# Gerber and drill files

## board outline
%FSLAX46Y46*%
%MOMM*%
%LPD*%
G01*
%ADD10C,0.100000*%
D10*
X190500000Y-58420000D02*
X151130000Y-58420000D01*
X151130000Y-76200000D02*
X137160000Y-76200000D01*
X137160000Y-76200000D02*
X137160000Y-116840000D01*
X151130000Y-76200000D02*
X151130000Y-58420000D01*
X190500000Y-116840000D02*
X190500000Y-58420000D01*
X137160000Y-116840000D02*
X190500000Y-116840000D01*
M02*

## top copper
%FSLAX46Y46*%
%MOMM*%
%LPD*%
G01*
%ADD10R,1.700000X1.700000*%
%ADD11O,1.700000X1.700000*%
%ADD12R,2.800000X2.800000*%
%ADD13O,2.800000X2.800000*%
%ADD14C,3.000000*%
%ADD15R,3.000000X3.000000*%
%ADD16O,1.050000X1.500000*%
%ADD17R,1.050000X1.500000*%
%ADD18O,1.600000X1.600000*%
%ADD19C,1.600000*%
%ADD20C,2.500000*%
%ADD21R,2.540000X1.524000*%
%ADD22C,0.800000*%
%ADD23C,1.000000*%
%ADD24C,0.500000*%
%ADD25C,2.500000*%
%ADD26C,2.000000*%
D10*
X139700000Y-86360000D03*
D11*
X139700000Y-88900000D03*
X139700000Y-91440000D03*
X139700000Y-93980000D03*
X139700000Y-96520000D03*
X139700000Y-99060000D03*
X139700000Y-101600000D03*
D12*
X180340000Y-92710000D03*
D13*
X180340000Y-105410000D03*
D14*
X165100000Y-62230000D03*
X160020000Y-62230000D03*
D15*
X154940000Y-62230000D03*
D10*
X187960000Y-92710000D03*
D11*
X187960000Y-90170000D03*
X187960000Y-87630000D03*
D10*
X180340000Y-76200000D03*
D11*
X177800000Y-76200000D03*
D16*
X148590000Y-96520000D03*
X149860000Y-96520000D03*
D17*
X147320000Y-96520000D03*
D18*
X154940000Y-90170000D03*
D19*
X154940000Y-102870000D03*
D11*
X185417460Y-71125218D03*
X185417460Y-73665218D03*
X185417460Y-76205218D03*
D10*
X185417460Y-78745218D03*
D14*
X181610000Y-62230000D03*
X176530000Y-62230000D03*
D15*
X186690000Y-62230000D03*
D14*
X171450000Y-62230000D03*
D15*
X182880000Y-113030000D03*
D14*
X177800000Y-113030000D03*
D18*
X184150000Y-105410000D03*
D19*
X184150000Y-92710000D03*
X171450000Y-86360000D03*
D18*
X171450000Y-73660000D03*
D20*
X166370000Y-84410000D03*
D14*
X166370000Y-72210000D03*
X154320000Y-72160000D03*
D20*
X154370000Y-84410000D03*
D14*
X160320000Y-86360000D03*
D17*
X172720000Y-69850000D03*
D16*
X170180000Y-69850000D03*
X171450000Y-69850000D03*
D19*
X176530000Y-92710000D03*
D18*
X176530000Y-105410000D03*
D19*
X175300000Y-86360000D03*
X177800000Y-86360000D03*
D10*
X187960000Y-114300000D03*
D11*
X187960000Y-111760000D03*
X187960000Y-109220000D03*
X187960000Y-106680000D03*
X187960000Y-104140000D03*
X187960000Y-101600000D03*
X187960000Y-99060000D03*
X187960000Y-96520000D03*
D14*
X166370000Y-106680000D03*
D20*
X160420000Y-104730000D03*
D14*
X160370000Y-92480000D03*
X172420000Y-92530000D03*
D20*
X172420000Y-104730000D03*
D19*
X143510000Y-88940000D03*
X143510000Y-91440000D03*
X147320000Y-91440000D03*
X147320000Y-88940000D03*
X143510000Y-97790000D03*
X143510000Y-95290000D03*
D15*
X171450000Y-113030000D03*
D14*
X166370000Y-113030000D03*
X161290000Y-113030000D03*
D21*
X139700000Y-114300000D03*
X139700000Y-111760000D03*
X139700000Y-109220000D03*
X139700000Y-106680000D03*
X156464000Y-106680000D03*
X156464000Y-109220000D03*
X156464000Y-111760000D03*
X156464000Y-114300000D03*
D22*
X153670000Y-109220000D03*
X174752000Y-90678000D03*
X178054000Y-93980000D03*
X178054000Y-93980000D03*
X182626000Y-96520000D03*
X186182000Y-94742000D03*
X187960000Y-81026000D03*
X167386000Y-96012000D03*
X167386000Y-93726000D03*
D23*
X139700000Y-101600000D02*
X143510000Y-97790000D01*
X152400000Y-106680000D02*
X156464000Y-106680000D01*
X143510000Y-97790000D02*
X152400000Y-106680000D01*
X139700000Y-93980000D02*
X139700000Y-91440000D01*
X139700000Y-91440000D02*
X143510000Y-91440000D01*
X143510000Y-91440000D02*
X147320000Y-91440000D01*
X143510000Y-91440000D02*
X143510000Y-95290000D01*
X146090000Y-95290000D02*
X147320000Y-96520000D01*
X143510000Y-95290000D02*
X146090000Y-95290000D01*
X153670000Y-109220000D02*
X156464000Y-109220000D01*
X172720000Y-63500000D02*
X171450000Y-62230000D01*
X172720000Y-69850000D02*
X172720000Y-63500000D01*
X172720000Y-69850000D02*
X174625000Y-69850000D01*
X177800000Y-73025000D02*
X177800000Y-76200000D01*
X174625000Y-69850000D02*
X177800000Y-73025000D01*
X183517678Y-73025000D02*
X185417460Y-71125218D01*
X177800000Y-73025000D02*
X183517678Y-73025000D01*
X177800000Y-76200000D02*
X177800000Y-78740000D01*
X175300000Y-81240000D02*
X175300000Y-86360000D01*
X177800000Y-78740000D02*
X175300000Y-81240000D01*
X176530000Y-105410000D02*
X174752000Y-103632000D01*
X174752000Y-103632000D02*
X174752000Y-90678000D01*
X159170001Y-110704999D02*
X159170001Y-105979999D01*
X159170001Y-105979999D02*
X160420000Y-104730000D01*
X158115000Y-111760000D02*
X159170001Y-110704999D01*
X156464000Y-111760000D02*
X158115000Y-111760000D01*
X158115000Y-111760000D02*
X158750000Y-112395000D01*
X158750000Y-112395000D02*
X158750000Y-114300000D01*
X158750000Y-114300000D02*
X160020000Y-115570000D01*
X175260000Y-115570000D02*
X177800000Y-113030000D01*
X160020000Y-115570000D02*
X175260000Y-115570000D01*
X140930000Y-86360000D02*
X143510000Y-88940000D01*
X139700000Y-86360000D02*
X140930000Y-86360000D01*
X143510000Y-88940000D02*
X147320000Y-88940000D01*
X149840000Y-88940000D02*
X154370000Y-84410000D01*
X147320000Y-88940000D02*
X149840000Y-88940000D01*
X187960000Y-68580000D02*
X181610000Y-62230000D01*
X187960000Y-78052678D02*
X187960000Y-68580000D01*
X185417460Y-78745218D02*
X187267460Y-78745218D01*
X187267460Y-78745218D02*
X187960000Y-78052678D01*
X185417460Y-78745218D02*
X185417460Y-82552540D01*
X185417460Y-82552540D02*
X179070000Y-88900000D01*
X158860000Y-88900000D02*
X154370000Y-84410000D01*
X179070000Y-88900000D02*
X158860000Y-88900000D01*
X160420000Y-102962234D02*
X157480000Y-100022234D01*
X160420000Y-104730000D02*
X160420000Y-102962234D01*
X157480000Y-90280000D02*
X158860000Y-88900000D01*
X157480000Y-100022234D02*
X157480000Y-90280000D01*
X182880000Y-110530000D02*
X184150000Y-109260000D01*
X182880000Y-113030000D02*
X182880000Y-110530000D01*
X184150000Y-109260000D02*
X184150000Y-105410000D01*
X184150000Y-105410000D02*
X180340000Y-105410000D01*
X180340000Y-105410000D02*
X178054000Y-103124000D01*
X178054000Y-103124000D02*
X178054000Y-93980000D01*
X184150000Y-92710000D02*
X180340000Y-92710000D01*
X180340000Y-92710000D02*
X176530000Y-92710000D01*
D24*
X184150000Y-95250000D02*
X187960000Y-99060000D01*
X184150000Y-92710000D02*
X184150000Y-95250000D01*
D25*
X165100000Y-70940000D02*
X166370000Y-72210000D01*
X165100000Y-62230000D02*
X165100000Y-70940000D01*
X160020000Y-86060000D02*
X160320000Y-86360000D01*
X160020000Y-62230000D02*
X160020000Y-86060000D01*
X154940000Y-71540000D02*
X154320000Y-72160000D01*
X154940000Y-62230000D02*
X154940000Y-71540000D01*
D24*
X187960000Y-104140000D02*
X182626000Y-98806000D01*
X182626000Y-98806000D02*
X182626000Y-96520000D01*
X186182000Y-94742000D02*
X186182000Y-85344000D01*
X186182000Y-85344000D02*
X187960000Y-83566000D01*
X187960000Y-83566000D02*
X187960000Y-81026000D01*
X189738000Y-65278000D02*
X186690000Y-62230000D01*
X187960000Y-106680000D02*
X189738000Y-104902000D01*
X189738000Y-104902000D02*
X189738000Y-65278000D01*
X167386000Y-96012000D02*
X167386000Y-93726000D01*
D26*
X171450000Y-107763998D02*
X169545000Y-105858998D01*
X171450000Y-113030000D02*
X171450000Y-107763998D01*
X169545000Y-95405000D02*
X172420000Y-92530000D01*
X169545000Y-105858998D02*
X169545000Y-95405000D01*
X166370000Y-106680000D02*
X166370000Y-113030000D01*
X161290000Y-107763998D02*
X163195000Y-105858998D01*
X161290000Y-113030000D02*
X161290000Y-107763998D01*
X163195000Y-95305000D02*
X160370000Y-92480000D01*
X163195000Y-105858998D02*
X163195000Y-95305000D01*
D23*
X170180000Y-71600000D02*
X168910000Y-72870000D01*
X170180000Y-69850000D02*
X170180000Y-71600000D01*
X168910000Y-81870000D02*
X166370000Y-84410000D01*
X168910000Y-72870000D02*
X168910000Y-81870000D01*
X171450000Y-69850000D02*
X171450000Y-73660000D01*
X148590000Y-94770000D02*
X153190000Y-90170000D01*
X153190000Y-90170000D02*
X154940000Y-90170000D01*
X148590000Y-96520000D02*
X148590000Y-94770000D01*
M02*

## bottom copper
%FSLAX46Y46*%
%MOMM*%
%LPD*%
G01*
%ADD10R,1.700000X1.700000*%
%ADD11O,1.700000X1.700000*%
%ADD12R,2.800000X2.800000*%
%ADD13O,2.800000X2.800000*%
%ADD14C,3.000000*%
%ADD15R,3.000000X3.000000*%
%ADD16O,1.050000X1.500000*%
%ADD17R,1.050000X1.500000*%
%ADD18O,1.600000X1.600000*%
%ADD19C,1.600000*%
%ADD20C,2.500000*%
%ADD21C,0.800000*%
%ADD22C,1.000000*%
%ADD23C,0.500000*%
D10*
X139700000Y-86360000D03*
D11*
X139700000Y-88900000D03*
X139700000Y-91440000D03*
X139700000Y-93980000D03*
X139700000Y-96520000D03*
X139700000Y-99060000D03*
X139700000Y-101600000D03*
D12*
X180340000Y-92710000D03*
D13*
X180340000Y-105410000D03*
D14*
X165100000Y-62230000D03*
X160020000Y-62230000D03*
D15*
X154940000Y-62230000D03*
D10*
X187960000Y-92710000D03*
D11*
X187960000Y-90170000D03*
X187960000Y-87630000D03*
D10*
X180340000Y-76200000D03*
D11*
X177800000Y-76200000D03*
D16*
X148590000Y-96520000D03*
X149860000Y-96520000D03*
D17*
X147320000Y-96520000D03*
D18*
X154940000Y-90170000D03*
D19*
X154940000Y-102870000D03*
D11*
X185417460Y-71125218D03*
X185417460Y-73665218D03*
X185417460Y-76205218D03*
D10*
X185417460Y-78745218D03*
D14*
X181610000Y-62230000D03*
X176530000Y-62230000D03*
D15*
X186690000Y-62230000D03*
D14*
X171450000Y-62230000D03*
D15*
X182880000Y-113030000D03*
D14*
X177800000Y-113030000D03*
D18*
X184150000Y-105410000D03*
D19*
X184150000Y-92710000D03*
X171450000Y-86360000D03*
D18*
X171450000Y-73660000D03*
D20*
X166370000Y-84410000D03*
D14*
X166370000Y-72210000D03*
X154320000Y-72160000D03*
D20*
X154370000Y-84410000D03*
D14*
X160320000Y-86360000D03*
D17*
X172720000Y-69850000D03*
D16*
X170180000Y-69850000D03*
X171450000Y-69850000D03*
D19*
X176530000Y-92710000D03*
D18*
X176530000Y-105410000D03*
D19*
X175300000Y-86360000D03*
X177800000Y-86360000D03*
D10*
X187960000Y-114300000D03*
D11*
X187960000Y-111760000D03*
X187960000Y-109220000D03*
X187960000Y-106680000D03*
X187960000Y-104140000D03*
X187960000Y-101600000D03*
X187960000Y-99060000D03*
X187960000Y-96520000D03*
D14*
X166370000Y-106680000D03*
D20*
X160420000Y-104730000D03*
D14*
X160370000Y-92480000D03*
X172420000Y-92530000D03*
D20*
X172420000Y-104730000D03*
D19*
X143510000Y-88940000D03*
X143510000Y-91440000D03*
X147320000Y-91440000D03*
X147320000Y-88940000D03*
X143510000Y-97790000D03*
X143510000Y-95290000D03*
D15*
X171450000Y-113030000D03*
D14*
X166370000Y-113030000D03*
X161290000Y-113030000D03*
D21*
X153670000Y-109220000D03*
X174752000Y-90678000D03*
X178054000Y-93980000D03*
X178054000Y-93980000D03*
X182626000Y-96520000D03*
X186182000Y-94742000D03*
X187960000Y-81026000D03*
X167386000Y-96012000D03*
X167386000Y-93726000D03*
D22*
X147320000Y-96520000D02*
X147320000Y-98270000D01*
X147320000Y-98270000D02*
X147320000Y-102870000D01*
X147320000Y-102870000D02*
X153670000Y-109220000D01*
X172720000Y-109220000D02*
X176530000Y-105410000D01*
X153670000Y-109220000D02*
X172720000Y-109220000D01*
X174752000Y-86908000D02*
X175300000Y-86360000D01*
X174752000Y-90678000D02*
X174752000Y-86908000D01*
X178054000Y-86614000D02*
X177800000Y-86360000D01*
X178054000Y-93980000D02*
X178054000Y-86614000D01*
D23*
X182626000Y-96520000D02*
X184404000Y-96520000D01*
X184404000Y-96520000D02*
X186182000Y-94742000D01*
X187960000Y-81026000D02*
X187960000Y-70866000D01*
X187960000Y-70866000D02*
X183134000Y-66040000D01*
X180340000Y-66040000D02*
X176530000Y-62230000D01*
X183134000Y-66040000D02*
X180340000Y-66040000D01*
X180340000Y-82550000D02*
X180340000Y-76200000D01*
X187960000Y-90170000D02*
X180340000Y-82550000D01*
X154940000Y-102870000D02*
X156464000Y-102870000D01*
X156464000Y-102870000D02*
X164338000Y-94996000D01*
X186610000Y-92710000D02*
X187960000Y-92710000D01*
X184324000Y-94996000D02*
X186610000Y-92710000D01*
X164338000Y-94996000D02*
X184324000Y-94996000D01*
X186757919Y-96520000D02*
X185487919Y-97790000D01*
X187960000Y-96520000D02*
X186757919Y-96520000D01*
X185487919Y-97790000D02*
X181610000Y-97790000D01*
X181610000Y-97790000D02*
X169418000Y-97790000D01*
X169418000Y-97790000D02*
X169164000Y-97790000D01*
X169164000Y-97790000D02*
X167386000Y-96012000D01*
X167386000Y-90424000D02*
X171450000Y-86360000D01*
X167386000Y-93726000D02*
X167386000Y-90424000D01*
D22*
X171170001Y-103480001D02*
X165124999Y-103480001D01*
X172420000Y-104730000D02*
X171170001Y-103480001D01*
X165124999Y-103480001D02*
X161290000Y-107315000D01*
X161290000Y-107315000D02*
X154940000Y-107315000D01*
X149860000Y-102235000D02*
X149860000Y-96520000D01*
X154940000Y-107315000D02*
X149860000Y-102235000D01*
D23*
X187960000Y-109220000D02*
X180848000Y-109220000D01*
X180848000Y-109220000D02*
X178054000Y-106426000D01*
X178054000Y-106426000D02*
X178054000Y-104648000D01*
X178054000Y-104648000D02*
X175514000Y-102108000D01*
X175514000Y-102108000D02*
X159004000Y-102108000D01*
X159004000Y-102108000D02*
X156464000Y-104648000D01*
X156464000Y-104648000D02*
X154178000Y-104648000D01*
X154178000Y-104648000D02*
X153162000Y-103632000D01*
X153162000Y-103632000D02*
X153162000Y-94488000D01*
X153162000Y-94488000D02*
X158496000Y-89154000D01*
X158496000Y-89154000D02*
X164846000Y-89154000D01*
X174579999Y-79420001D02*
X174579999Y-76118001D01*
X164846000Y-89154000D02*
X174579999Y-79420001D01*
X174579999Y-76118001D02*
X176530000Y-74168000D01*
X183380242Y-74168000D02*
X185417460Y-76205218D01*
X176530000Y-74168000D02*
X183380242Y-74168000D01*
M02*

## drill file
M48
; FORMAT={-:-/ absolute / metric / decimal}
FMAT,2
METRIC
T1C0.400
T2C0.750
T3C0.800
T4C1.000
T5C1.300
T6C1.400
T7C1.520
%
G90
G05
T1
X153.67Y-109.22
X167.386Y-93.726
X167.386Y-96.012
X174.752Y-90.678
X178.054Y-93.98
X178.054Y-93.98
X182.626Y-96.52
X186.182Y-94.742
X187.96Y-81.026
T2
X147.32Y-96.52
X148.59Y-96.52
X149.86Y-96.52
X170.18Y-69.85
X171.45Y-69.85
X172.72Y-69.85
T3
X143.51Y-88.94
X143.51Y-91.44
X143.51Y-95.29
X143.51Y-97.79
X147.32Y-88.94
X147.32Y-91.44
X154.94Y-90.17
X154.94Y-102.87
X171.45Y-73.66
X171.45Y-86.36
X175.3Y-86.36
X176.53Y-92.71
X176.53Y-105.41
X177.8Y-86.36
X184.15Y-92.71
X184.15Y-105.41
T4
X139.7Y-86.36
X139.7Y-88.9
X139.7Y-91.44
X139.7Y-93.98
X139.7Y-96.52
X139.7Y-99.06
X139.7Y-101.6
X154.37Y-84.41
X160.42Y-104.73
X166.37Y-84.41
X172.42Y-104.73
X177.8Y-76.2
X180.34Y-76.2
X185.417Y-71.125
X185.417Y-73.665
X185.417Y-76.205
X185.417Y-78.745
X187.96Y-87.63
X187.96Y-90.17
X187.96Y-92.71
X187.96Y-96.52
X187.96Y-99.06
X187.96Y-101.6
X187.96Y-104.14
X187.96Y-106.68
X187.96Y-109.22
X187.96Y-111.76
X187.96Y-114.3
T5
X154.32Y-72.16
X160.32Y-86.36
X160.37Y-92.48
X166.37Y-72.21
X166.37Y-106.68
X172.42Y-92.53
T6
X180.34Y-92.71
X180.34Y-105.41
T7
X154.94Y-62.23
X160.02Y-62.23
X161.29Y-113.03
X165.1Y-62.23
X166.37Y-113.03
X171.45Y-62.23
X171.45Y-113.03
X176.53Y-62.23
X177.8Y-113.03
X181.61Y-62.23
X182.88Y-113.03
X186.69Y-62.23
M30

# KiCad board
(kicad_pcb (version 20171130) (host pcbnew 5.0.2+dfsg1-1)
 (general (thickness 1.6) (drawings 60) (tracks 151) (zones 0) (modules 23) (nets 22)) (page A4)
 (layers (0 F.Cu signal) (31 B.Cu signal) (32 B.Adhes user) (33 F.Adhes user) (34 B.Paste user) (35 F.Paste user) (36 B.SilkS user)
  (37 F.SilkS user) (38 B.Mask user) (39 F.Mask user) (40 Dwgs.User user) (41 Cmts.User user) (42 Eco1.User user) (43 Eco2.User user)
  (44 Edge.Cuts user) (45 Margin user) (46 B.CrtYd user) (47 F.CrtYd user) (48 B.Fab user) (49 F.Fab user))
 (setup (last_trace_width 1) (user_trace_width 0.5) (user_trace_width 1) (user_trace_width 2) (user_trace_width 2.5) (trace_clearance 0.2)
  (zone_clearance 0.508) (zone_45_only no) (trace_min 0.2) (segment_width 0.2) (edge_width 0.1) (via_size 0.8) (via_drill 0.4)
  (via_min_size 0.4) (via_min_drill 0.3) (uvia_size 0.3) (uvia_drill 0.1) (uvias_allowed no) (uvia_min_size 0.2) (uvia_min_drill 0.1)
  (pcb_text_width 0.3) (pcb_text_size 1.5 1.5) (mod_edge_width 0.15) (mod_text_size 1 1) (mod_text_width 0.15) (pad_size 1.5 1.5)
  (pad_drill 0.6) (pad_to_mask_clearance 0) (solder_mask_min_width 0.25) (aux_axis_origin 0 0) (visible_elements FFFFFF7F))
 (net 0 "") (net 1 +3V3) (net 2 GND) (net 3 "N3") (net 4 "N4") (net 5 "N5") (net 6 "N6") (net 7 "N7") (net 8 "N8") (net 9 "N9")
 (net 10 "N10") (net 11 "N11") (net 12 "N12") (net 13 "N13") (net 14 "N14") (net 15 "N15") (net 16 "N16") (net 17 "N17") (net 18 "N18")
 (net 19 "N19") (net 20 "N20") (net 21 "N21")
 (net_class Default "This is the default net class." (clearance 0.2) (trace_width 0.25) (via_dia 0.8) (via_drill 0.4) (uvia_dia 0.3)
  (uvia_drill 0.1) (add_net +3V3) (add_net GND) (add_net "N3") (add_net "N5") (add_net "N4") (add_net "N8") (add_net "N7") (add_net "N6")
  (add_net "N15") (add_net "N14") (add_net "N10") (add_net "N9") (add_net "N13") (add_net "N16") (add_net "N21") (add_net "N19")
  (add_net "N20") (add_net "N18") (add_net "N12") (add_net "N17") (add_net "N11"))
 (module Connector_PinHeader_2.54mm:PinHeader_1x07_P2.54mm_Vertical (layer F.Cu) (at 139.7 86.36)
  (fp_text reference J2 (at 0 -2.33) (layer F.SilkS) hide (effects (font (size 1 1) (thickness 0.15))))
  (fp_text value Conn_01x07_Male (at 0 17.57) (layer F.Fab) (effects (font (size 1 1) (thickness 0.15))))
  (pad 1 thru_hole rect (at 0 0) (size 1.7 1.7) (drill 1) (layers *.Cu *.Mask) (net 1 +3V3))
  (pad 2 thru_hole oval (at 0 2.54) (size 1.7 1.7) (drill 1) (layers *.Cu *.Mask))
  (pad 3 thru_hole oval (at 0 5.08) (size 1.7 1.7) (drill 1) (layers *.Cu *.Mask) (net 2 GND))
  (pad 4 thru_hole oval (at 0 7.62) (size 1.7 1.7) (drill 1) (layers *.Cu *.Mask) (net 2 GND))
  (pad 5 thru_hole oval (at 0 10.16) (size 1.7 1.7) (drill 1) (layers *.Cu *.Mask))
  (pad 6 thru_hole oval (at 0 12.7) (size 1.7 1.7) (drill 1) (layers *.Cu *.Mask))
  (pad 7 thru_hole oval (at 0 15.24) (size 1.7 1.7) (drill 1) (layers *.Cu *.Mask) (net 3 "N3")))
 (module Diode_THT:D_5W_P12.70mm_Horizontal (layer F.Cu) (at 180.34 92.71 270)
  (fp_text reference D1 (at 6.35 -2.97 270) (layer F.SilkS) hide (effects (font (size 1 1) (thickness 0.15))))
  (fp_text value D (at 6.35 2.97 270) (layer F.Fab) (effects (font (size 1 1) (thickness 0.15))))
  (pad 1 thru_hole rect (at 0 0 270) (size 2.8 2.8) (drill 1.4) (layers *.Cu *.Mask) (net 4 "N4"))
  (pad 2 thru_hole oval (at 12.7 0 270) (size 2.8 2.8) (drill 1.4) (layers *.Cu *.Mask) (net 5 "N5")))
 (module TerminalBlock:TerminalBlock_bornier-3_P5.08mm (layer F.Cu) (at 154.94 62.23)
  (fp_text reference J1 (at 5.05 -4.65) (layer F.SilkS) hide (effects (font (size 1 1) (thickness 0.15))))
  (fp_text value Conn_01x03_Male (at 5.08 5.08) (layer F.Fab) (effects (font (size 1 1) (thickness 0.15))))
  (pad 3 thru_hole circle (at 10.16 0) (size 3 3) (drill 1.52) (layers *.Cu *.Mask) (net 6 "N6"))
  (pad 2 thru_hole circle (at 5.08 0) (size 3 3) (drill 1.52) (layers *.Cu *.Mask) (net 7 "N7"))
  (pad 1 thru_hole rect (at 0 0) (size 3 3) (drill 1.52) (layers *.Cu *.Mask) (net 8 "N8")))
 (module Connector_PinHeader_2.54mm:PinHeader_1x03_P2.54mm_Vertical (layer F.Cu) (at 187.96 92.71 180)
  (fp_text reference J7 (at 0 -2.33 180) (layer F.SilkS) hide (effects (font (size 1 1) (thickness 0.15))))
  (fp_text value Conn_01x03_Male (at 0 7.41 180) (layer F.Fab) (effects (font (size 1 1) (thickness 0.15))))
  (pad 1 thru_hole rect (at 0 0 180) (size 1.7 1.7) (drill 1) (layers *.Cu *.Mask) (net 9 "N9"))
  (pad 2 thru_hole oval (at 0 2.54 180) (size 1.7 1.7) (drill 1) (layers *.Cu *.Mask) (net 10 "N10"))
  (pad 3 thru_hole oval (at 0 5.08 180) (size 1.7 1.7) (drill 1) (layers *.Cu *.Mask)))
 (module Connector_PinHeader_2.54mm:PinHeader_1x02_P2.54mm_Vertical (layer F.Cu) (at 180.34 76.2 270)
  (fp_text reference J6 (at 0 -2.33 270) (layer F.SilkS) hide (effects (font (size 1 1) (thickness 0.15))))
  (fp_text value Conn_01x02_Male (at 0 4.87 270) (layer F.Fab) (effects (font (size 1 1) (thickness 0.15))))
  (pad 1 thru_hole rect (at 0 0 270) (size 1.7 1.7) (drill 1) (layers *.Cu *.Mask) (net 10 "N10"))
  (pad 2 thru_hole oval (at 0 2.54 270) (size 1.7 1.7) (drill 1) (layers *.Cu *.Mask) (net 2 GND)))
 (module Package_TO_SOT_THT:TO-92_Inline (layer F.Cu) (at 147.32 96.52)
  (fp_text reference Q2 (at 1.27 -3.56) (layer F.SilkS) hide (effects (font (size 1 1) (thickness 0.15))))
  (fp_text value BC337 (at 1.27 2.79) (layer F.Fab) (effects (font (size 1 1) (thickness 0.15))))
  (pad 2 thru_hole oval (at 1.27 0) (size 1.05 1.5) (drill 0.75) (layers *.Cu *.Mask) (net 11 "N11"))
  (pad 3 thru_hole oval (at 2.54 0) (size 1.05 1.5) (drill 0.75) (layers *.Cu *.Mask) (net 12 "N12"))
  (pad 1 thru_hole rect (at 0 0) (size 1.05 1.5) (drill 0.75) (layers *.Cu *.Mask) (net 2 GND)))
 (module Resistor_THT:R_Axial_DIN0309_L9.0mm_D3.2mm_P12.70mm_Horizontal (layer F.Cu) (at 154.94 102.87 90)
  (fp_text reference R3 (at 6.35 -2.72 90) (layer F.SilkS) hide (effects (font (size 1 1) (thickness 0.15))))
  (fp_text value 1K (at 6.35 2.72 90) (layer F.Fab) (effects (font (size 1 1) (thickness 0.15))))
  (pad 2 thru_hole oval (at 12.7 0 90) (size 1.6 1.6) (drill 0.8) (layers *.Cu *.Mask) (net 11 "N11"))
  (pad 1 thru_hole circle (at 0 0 90) (size 1.6 1.6) (drill 0.8) (layers *.Cu *.Mask) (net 9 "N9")))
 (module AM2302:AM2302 (layer F.Cu) (at 185.42 74.93 90)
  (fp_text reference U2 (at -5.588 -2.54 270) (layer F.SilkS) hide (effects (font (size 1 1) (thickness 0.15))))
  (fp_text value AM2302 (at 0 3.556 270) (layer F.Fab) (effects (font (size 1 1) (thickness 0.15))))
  (pad 4 thru_hole oval (at 3.804782 -0.00254 180) (size 1.7 1.7) (drill 1) (layers *.Cu *.Mask) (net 2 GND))
  (pad 3 thru_hole oval (at 1.264782 -0.00254 180) (size 1.7 1.7) (drill 1) (layers *.Cu *.Mask))
  (pad 2 thru_hole oval (at -1.275218 -0.00254 180) (size 1.7 1.7) (drill 1) (layers *.Cu *.Mask) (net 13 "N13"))
  (pad 1 thru_hole rect (at -3.815218 -0.00254) (size 1.7 1.7) (drill 1) (layers *.Cu *.Mask) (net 1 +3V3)))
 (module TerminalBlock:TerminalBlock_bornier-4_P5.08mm (layer F.Cu) (at 186.69 62.23 180)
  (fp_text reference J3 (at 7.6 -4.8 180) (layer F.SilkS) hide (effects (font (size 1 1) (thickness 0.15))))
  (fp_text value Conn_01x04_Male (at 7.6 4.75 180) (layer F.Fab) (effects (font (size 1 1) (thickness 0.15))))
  (pad 2 thru_hole circle (at 5.08 0 180) (size 3 3) (drill 1.52) (layers *.Cu *.Mask) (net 1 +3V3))
  (pad 3 thru_hole circle (at 10.16 0 180) (size 3 3) (drill 1.52) (layers *.Cu *.Mask) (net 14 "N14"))
  (pad 1 thru_hole rect (at 0 0 180) (size 3 3) (drill 1.52) (layers *.Cu *.Mask) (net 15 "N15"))
  (pad 4 thru_hole circle (at 15.24 0 180) (size 3 3) (drill 1.52) (layers *.Cu *.Mask) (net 2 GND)))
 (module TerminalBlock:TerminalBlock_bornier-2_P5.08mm (layer F.Cu) (at 182.88 113.03 180)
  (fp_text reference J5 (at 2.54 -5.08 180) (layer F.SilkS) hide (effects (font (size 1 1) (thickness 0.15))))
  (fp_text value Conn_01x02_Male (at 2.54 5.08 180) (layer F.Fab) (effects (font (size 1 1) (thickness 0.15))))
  (pad 1 thru_hole rect (at 0 0 180) (size 3 3) (drill 1.52) (layers *.Cu *.Mask) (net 5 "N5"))
  (pad 2 thru_hole circle (at 5.08 0 180) (size 3 3) (drill 1.52) (layers *.Cu *.Mask) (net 1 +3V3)))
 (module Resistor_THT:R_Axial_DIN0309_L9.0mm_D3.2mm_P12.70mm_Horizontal (layer F.Cu) (at 184.15 92.71 270)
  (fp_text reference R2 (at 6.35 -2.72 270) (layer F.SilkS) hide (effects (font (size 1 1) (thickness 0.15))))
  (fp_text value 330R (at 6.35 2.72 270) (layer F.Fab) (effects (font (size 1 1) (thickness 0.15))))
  (pad 2 thru_hole oval (at 12.7 0 270) (size 1.6 1.6) (drill 0.8) (layers *.Cu *.Mask) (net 5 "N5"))
  (pad 1 thru_hole circle (at 0 0 270) (size 1.6 1.6) (drill 0.8) (layers *.Cu *.Mask) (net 4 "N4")))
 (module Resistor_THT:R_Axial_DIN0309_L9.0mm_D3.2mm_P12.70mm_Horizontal (layer F.Cu) (at 171.45 86.36 90)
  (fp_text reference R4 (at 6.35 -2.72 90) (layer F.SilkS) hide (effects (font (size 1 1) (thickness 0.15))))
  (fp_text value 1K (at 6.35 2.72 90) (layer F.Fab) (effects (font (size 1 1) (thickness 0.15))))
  (pad 1 thru_hole circle (at 0 0 90) (size 1.6 1.6) (drill 0.8) (layers *.Cu *.Mask) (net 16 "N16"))
  (pad 2 thru_hole oval (at 12.7 0 90) (size 1.6 1.6) (drill 0.8) (layers *.Cu *.Mask) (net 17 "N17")))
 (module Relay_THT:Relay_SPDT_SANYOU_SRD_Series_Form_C (layer F.Cu) (at 160.32 86.36 90)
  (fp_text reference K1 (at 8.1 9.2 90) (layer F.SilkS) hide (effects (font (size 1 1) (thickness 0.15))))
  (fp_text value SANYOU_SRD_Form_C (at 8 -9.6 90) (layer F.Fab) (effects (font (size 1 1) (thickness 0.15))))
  (pad 2 thru_hole circle (at 1.95 6.05 180) (size 2.5 2.5) (drill 1) (layers *.Cu *.Mask) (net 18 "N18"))
  (pad 3 thru_hole circle (at 14.15 6.05 180) (size 3 3) (drill 1.3) (layers *.Cu *.Mask) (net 6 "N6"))
  (pad 4 thru_hole circle (at 14.2 -6 180) (size 3 3) (drill 1.3) (layers *.Cu *.Mask) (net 8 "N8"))
  (pad 5 thru_hole circle (at 1.95 -5.95 180) (size 2.5 2.5) (drill 1) (layers *.Cu *.Mask) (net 1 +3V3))
  (pad 1 thru_hole circle (at 0 0 180) (size 3 3) (drill 1.3) (layers *.Cu *.Mask) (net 7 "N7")))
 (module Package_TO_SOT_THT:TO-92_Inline (layer F.Cu) (at 172.72 69.85 180)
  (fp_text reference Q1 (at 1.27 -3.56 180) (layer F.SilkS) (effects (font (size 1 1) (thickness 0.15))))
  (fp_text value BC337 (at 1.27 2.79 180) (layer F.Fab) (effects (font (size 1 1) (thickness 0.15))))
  (pad 1 thru_hole rect (at 0 0 180) (size 1.05 1.5) (drill 0.75) (layers *.Cu *.Mask) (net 2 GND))
  (pad 3 thru_hole oval (at 2.54 0 180) (size 1.05 1.5) (drill 0.75) (layers *.Cu *.Mask) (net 18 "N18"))
  (pad 2 thru_hole oval (at 1.27 0 180) (size 1.05 1.5) (drill 0.75) (layers *.Cu *.Mask) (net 17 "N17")))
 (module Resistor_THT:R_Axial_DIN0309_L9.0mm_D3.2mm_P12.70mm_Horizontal (layer F.Cu) (at 176.53 92.71 270)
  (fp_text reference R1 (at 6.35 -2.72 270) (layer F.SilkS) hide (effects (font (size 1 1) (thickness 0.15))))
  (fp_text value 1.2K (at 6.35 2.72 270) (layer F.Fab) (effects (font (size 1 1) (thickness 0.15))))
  (pad 1 thru_hole circle (at 0 0 270) (size 1.6 1.6) (drill 0.8) (layers *.Cu *.Mask) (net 4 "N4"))
  (pad 2 thru_hole oval (at 12.7 0 270) (size 1.6 1.6) (drill 0.8) (layers *.Cu *.Mask) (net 2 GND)))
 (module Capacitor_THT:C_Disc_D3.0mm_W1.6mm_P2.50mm (layer F.Cu) (at 177.8 86.36 180)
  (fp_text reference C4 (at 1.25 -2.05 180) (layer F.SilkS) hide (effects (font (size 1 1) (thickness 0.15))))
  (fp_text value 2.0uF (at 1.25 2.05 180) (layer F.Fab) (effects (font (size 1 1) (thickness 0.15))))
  (pad 2 thru_hole circle (at 2.5 0 180) (size 1.6 1.6) (drill 0.8) (layers *.Cu *.Mask) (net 2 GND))
  (pad 1 thru_hole circle (at 0 0 180) (size 1.6 1.6) (drill 0.8) (layers *.Cu *.Mask) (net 5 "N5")))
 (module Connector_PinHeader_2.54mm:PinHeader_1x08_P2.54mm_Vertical (layer F.Cu) (at 187.96 114.3 180)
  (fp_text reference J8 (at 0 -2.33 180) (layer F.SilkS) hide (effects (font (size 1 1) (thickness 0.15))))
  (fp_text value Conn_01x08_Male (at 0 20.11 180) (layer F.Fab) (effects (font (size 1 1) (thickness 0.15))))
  (pad 1 thru_hole rect (at 0 0 180) (size 1.7 1.7) (drill 1) (layers *.Cu *.Mask))
  (pad 2 thru_hole oval (at 0 2.54 180) (size 1.7 1.7) (drill 1) (layers *.Cu *.Mask))
  (pad 3 thru_hole oval (at 0 5.08 180) (size 1.7 1.7) (drill 1) (layers *.Cu *.Mask) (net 13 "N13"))
  (pad 4 thru_hole oval (at 0 7.62 180) (size 1.7 1.7) (drill 1) (layers *.Cu *.Mask) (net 15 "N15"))
  (pad 5 thru_hole oval (at 0 10.16 180) (size 1.7 1.7) (drill 1) (layers *.Cu *.Mask) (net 14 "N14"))
  (pad 6 thru_hole oval (at 0 12.7 180) (size 1.7 1.7) (drill 1) (layers *.Cu *.Mask))
  (pad 7 thru_hole oval (at 0 15.24 180) (size 1.7 1.7) (drill 1) (layers *.Cu *.Mask) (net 4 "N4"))
  (pad 8 thru_hole oval (at 0 17.78 180) (size 1.7 1.7) (drill 1) (layers *.Cu *.Mask) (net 16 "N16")))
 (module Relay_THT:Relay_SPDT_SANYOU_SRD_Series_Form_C (layer F.Cu) (at 166.37 106.68 90)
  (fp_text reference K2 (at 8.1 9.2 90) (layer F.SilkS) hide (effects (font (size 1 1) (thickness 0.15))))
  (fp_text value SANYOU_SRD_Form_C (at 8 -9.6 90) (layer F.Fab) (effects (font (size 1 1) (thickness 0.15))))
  (pad 1 thru_hole circle (at 0 0 180) (size 3 3) (drill 1.3) (layers *.Cu *.Mask) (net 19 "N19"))
  (pad 5 thru_hole circle (at 1.95 -5.95 180) (size 2.5 2.5) (drill 1) (layers *.Cu *.Mask) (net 1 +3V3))
  (pad 4 thru_hole circle (at 14.2 -6 180) (size 3 3) (drill 1.3) (layers *.Cu *.Mask) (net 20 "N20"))
  (pad 3 thru_hole circle (at 14.15 6.05 180) (size 3 3) (drill 1.3) (layers *.Cu *.Mask) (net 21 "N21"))
  (pad 2 thru_hole circle (at 1.95 6.05 180) (size 2.5 2.5) (drill 1) (layers *.Cu *.Mask) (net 12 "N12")))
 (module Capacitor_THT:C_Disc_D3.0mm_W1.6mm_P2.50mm (layer F.Cu) (at 143.51 88.94 270)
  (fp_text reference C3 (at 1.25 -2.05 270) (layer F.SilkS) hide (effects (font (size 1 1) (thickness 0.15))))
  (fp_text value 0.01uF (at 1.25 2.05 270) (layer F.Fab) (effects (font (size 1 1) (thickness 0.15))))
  (pad 1 thru_hole circle (at 0 0 270) (size 1.6 1.6) (drill 0.8) (layers *.Cu *.Mask) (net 1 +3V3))
  (pad 2 thru_hole circle (at 2.5 0 270) (size 1.6 1.6) (drill 0.8) (layers *.Cu *.Mask) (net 2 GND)))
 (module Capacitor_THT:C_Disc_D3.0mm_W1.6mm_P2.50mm (layer F.Cu) (at 147.32 88.94 270)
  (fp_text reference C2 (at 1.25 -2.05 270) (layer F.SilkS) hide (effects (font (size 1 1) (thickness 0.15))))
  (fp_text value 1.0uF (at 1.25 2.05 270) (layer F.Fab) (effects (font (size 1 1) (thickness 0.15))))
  (pad 2 thru_hole circle (at 2.5 0 270) (size 1.6 1.6) (drill 0.8) (layers *.Cu *.Mask) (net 2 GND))
  (pad 1 thru_hole circle (at 0 0 270) (size 1.6 1.6) (drill 0.8) (layers *.Cu *.Mask) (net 1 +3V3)))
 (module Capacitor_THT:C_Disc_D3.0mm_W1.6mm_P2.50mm (layer F.Cu) (at 143.51 97.79 90)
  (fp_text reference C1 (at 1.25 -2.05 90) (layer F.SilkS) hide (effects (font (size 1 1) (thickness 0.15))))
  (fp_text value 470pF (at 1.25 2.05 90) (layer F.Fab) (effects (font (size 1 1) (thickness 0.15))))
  (pad 1 thru_hole circle (at 0 0 90) (size 1.6 1.6) (drill 0.8) (layers *.Cu *.Mask) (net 3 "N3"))
  (pad 2 thru_hole circle (at 2.5 0 90) (size 1.6 1.6) (drill 0.8) (layers *.Cu *.Mask) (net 2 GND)))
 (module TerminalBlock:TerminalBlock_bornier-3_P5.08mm (layer F.Cu) (at 171.45 113.03 180)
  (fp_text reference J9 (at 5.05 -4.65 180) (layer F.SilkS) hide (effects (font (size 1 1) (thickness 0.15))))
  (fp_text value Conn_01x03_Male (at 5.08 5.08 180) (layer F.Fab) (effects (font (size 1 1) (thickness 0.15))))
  (pad 1 thru_hole rect (at 0 0 180) (size 3 3) (drill 1.52) (layers *.Cu *.Mask) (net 21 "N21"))
  (pad 2 thru_hole circle (at 5.08 0 180) (size 3 3) (drill 1.52) (layers *.Cu *.Mask) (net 19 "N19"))
  (pad 3 thru_hole circle (at 10.16 0 180) (size 3 3) (drill 1.52) (layers *.Cu *.Mask) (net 20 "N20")))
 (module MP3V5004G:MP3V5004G (layer F.Cu) (at 148.082 110.49)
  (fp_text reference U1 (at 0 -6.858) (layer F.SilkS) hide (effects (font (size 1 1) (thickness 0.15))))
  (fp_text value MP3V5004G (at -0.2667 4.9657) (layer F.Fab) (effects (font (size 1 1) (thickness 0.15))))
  (pad 8 smd rect (at -8.382 3.81) (size 2.54 1.524) (layers F.Cu F.Paste F.Mask))
  (pad 7 smd rect (at -8.382 1.27) (size 2.54 1.524) (layers F.Cu F.Paste F.Mask))
  (pad 6 smd rect (at -8.382 -1.27) (size 2.54 1.524) (layers F.Cu F.Paste F.Mask))
  (pad 5 smd rect (at -8.382 -3.81) (size 2.54 1.524) (layers F.Cu F.Paste F.Mask))
  (pad 4 smd rect (at 8.382 -3.81) (size 2.54 1.524) (layers F.Cu F.Paste F.Mask) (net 3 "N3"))
  (pad 3 smd rect (at 8.382 -1.27) (size 2.54 1.524) (layers F.Cu F.Paste F.Mask) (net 2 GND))
  (pad 2 smd rect (at 8.382 1.27) (size 2.54 1.524) (layers F.Cu F.Paste F.Mask) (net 1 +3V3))
  (pad 1 smd rect (at 8.382 3.81) (size 2.54 1.524) (layers F.Cu F.Paste F.Mask)))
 (gr_line (start 190.5 58.42) (end 151.13 58.42) (layer Edge.Cuts) (width 0.1))
 (gr_line (start 151.13 76.2) (end 137.16 76.2) (layer Edge.Cuts) (width 0.1))
 (gr_line (start 137.16 76.2) (end 137.16 116.84) (layer Edge.Cuts) (width 0.1))
 (gr_line (start 151.13 76.2) (end 151.13 58.42) (layer Edge.Cuts) (width 0.1))
 (gr_line (start 190.5 116.84) (end 190.5 58.42) (layer Edge.Cuts) (width 0.1))
 (gr_line (start 137.16 116.84) (end 190.5 116.84) (layer Edge.Cuts) (width 0.1))
 (segment (start 139.7 101.6) (end 143.51 97.79) (width 1) (layer F.Cu) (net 3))
 (segment (start 152.4 106.68) (end 156.464 106.68) (width 1) (layer F.Cu) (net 3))
 (segment (start 143.51 97.79) (end 152.4 106.68) (width 1) (layer F.Cu) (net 3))
 (segment (start 139.7 93.98) (end 139.7 91.44) (width 1) (layer F.Cu) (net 2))
 (segment (start 139.7 91.44) (end 143.51 91.44) (width 1) (layer F.Cu) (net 2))
 (segment (start 143.51 91.44) (end 147.32 91.44) (width 1) (layer F.Cu) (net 2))
 (segment (start 143.51 91.44) (end 143.51 95.29) (width 1) (layer F.Cu) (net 2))
 (segment (start 146.09 95.29) (end 147.32 96.52) (width 1) (layer F.Cu) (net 2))
 (segment (start 143.51 95.29) (end 146.09 95.29) (width 1) (layer F.Cu) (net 2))
 (segment (start 147.32 96.52) (end 147.32 98.27) (width 1) (layer B.Cu) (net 2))
 (segment (start 147.32 98.27) (end 147.32 102.87) (width 1) (layer B.Cu) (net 2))
 (via (at 153.67 109.22) (size 0.8) (drill 0.4) (layers F.Cu B.Cu) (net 2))
 (segment (start 147.32 102.87) (end 153.67 109.22) (width 1) (layer B.Cu) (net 2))
 (segment (start 153.67 109.22) (end 156.464 109.22) (width 1) (layer F.Cu) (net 2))
 (segment (start 172.72 109.22) (end 176.53 105.41) (width 1) (layer B.Cu) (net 2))
 (segment (start 153.67 109.22) (end 172.72 109.22) (width 1) (layer B.Cu) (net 2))
 (segment (start 172.72 63.5) (end 171.45 62.23) (width 1) (layer F.Cu) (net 2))
 (segment (start 172.72 69.85) (end 172.72 63.5) (width 1) (layer F.Cu) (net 2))
 (segment (start 172.72 69.85) (end 174.625 69.85) (width 1) (layer F.Cu) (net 2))
 (segment (start 177.8 73.025) (end 177.8 76.2) (width 1) (layer F.Cu) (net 2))
 (segment (start 174.625 69.85) (end 177.8 73.025) (width 1) (layer F.Cu) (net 2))
 (segment (start 183.517678 73.025) (end 185.41746 71.125218) (width 1) (layer F.Cu) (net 2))
 (segment (start 177.8 73.025) (end 183.517678 73.025) (width 1) (layer F.Cu) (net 2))
 (segment (start 177.8 76.2) (end 177.8 78.74) (width 1) (layer F.Cu) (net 2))
 (segment (start 175.3 81.24) (end 175.3 86.36) (width 1) (layer F.Cu) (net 2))
 (segment (start 177.8 78.74) (end 175.3 81.24) (width 1) (layer F.Cu) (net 2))
 (segment (start 176.53 105.41) (end 174.752 103.632) (width 1) (layer F.Cu) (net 2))
 (via (at 174.752 90.678) (size 0.8) (drill 0.4) (layers F.Cu B.Cu) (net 2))
 (segment (start 174.752 103.632) (end 174.752 90.678) (width 1) (layer F.Cu) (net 2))
 (segment (start 174.752 86.908) (end 175.3 86.36) (width 1) (layer B.Cu) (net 2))
 (segment (start 174.752 90.678) (end 174.752 86.908) (width 1) (layer B.Cu) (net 2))
 (segment (start 159.170001 110.704999) (end 159.170001 105.979999) (width 1) (layer F.Cu) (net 1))
 (segment (start 159.170001 105.979999) (end 160.42 104.73) (width 1) (layer F.Cu) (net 1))
 (segment (start 158.115 111.76) (end 159.170001 110.704999) (width 1) (layer F.Cu) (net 1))
 (segment (start 156.464 111.76) (end 158.115 111.76) (width 1) (layer F.Cu) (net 1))
 (segment (start 158.115 111.76) (end 158.75 112.395) (width 1) (layer F.Cu) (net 1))
 (segment (start 158.75 112.395) (end 158.75 114.3) (width 1) (layer F.Cu) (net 1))
 (segment (start 158.75 114.3) (end 160.02 115.57) (width 1) (layer F.Cu) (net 1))
 (segment (start 175.26 115.57) (end 177.8 113.03) (width 1) (layer F.Cu) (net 1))
 (segment (start 160.02 115.57) (end 175.26 115.57) (width 1) (layer F.Cu) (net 1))
 (segment (start 140.93 86.36) (end 143.51 88.94) (width 1) (layer F.Cu) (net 1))
 (segment (start 139.7 86.36) (end 140.93 86.36) (width 1) (layer F.Cu) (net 1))
 (segment (start 143.51 88.94) (end 147.32 88.94) (width 1) (layer F.Cu) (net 1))
 (segment (start 149.84 88.94) (end 154.37 84.41) (width 1) (layer F.Cu) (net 1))
 (segment (start 147.32 88.94) (end 149.84 88.94) (width 1) (layer F.Cu) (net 1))
 (segment (start 187.96 68.58) (end 181.61 62.23) (width 1) (layer F.Cu) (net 1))
 (segment (start 187.96 78.052678) (end 187.96 68.58) (width 1) (layer F.Cu) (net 1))
 (segment (start 185.41746 78.745218) (end 187.26746 78.745218) (width 1) (layer F.Cu) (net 1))
 (segment (start 187.26746 78.745218) (end 187.96 78.052678) (width 1) (layer F.Cu) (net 1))
 (segment (start 185.41746 78.745218) (end 185.41746 82.55254) (width 1) (layer F.Cu) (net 1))
 (segment (start 185.41746 82.55254) (end 179.07 88.9) (width 1) (layer F.Cu) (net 1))
 (segment (start 158.86 88.9) (end 154.37 84.41) (width 1) (layer F.Cu) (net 1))
 (segment (start 179.07 88.9) (end 158.86 88.9) (width 1) (layer F.Cu) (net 1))
 (segment (start 160.42 102.962234) (end 157.48 100.022234) (width 1) (layer F.Cu) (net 1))
 (segment (start 160.42 104.73) (end 160.42 102.962234) (width 1) (layer F.Cu) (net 1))
 (segment (start 157.48 90.28) (end 158.86 88.9) (width 1) (layer F.Cu) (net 1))
 (segment (start 157.48 100.022234) (end 157.48 90.28) (width 1) (layer F.Cu) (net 1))
 (segment (start 182.88 110.53) (end 184.15 109.26) (width 1) (layer F.Cu) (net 5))
 (segment (start 182.88 113.03) (end 182.88 110.53) (width 1) (layer F.Cu) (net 5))
 (segment (start 184.15 109.26) (end 184.15 105.41) (width 1) (layer F.Cu) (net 5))
 (segment (start 184.15 105.41) (end 180.34 105.41) (width 1) (layer F.Cu) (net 5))
 (via (at 178.054 93.98) (size 0.8) (drill 0.4) (layers F.Cu B.Cu) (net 5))
 (segment (start 180.34 105.41) (end 178.054 103.124) (width 1) (layer F.Cu) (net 5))
 (segment (start 178.054 103.124) (end 178.054 93.98) (width 1) (layer F.Cu) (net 5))
 (via (at 178.054 93.98) (size 0.8) (drill 0.4) (layers F.Cu B.Cu) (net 5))
 (segment (start 178.054 86.614) (end 177.8 86.36) (width 1) (layer B.Cu) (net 5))
 (segment (start 178.054 93.98) (end 178.054 86.614) (width 1) (layer B.Cu) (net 5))
 (segment (start 184.15 92.71) (end 180.34 92.71) (width 1) (layer F.Cu) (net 4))
 (segment (start 180.34 92.71) (end 176.53 92.71) (width 1) (layer F.Cu) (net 4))
 (segment (start 184.15 95.25) (end 187.96 99.06) (width 0.5) (layer F.Cu) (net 4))
 (segment (start 184.15 92.71) (end 184.15 95.25) (width 0.5) (layer F.Cu) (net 4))
 (segment (start 165.1 70.94) (end 166.37 72.21) (width 2.5) (layer F.Cu) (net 6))
 (segment (start 165.1 62.23) (end 165.1 70.94) (width 2.5) (layer F.Cu) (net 6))
 (segment (start 160.02 86.06) (end 160.32 86.36) (width 2.5) (layer F.Cu) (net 7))
 (segment (start 160.02 62.23) (end 160.02 86.06) (width 2.5) (layer F.Cu) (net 7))
 (segment (start 154.94 71.54) (end 154.32 72.16) (width 2.5) (layer F.Cu) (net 8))
 (segment (start 154.94 62.23) (end 154.94 71.54) (width 2.5) (layer F.Cu) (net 8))
 (segment (start 187.96 104.14) (end 182.626 98.806) (width 0.5) (layer F.Cu) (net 14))
 (via (at 182.626 96.52) (size 0.8) (drill 0.4) (layers F.Cu B.Cu) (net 14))
 (segment (start 182.626 98.806) (end 182.626 96.52) (width 0.5) (layer F.Cu) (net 14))
 (via (at 186.182 94.742) (size 0.8) (drill 0.4) (layers F.Cu B.Cu) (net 14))
 (segment (start 182.626 96.52) (end 184.404 96.52) (width 0.5) (layer B.Cu) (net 14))
 (segment (start 184.404 96.52) (end 186.182 94.742) (width 0.5) (layer B.Cu) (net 14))
 (segment (start 186.182 94.742) (end 186.182 85.344) (width 0.5) (layer F.Cu) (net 14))
 (segment (start 186.182 85.344) (end 187.96 83.566) (width 0.5) (layer F.Cu) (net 14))
 (via (at 187.96 81.026) (size 0.8) (drill 0.4) (layers F.Cu B.Cu) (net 14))
 (segment (start 187.96 83.566) (end 187.96 81.026) (width 0.5) (layer F.Cu) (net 14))
 (segment (start 187.96 81.026) (end 187.96 70.866) (width 0.5) (layer B.Cu) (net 14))
 (segment (start 187.96 70.866) (end 183.134 66.04) (width 0.5) (layer B.Cu) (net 14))
 (segment (start 180.34 66.04) (end 176.53 62.23) (width 0.5) (layer B.Cu) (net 14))
 (segment (start 183.134 66.04) (end 180.34 66.04) (width 0.5) (layer B.Cu) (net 14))
 (segment (start 189.738 65.278) (end 186.69 62.23) (width 0.5) (layer F.Cu) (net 15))
 (segment (start 187.96 106.68) (end 189.738 104.902) (width 0.5) (layer F.Cu) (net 15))
 (segment (start 189.738 104.902) (end 189.738 65.278) (width 0.5) (layer F.Cu) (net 15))
 (segment (start 180.34 82.55) (end 180.34 76.2) (width 0.5) (layer B.Cu) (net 10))
 (segment (start 187.96 90.17) (end 180.34 82.55) (width 0.5) (layer B.Cu) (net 10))
 (segment (start 154.94 102.87) (end 156.464 102.87) (width 0.5) (layer B.Cu) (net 9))
 (segment (start 156.464 102.87) (end 164.338 94.996) (width 0.5) (layer B.Cu) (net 9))
 (segment (start 186.61 92.71) (end 187.96 92.71) (width 0.5) (layer B.Cu) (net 9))
 (segment (start 184.324 94.996) (end 186.61 92.71) (width 0.5) (layer B.Cu) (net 9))
 (segment (start 164.338 94.996) (end 184.324 94.996) (width 0.5) (layer B.Cu) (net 9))
 (segment (start 186.757919 96.52) (end 185.487919 97.79) (width 0.5) (layer B.Cu) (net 16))
 (segment (start 187.96 96.52) (end 186.757919 96.52) (width 0.5) (layer B.Cu) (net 16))
 (segment (start 185.487919 97.79) (end 181.61 97.79) (width 0.5) (layer B.Cu) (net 16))
 (segment (start 181.61 97.79) (end 169.418 97.79) (width 0.5) (layer B.Cu) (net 16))
 (via (at 167.386 96.012) (size 0.8) (drill 0.4) (layers F.Cu B.Cu) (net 16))
 (segment (start 169.418 97.79) (end 169.164 97.79) (width 0.5) (layer B.Cu) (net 16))
 (segment (start 169.164 97.79) (end 167.386 96.012) (width 0.5) (layer B.Cu) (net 16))
 (via (at 167.386 93.726) (size 0.8) (drill 0.4) (layers F.Cu B.Cu) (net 16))
 (segment (start 167.386 96.012) (end 167.386 93.726) (width 0.5) (layer F.Cu) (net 16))
 (segment (start 167.386 90.424) (end 171.45 86.36) (width 0.5) (layer B.Cu) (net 16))
 (segment (start 167.386 93.726) (end 167.386 90.424) (width 0.5) (layer B.Cu) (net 16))
 (segment (start 171.45 107.763998) (end 169.545 105.858998) (width 2) (layer F.Cu) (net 21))
 (segment (start 171.45 113.03) (end 171.45 107.763998) (width 2) (layer F.Cu) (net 21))
 (segment (start 169.545 95.405) (end 172.42 92.53) (width 2) (layer F.Cu) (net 21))
 (segment (start 169.545 105.858998) (end 169.545 95.405) (width 2) (layer F.Cu) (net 21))
 (segment (start 166.37 106.68) (end 166.37 113.03) (width 2) (layer F.Cu) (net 19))
 (segment (start 161.29 107.763998) (end 163.195 105.858998) (width 2) (layer F.Cu) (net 20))
 (segment (start 161.29 113.03) (end 161.29 107.763998) (width 2) (layer F.Cu) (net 20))
 (segment (start 163.195 95.305) (end 160.37 92.48) (width 2) (layer F.Cu) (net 20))
 (segment (start 163.195 105.858998) (end 163.195 95.305) (width 2) (layer F.Cu) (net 20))
 (segment (start 170.18 71.6) (end 168.91 72.87) (width 1) (layer F.Cu) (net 18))
 (segment (start 170.18 69.85) (end 170.18 71.6) (width 1) (layer F.Cu) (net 18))
 (segment (start 168.91 81.87) (end 166.37 84.41) (width 1) (layer F.Cu) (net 18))
 (segment (start 168.91 72.87) (end 168.91 81.87) (width 1) (layer F.Cu) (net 18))
 (segment (start 171.170001 103.480001) (end 165.124999 103.480001) (width 1) (layer B.Cu) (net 12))
 (segment (start 172.42 104.73) (end 171.170001 103.480001) (width 1) (layer B.Cu) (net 12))
 (segment (start 165.124999 103.480001) (end 161.29 107.315) (width 1) (layer B.Cu) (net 12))
 (segment (start 161.29 107.315) (end 154.94 107.315) (width 1) (layer B.Cu) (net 12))
 (segment (start 149.86 102.235) (end 149.86 96.52) (width 1) (layer B.Cu) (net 12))
 (segment (start 154.94 107.315) (end 149.86 102.235) (width 1) (layer B.Cu) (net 12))
 (segment (start 171.45 69.85) (end 171.45 73.66) (width 1) (layer F.Cu) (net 17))
 (segment (start 148.59 94.77) (end 153.19 90.17) (width 1) (layer F.Cu) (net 11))
 (segment (start 153.19 90.17) (end 154.94 90.17) (width 1) (layer F.Cu) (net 11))
 (segment (start 148.59 96.52) (end 148.59 94.77) (width 1) (layer F.Cu) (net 11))
 (segment (start 187.96 109.22) (end 180.848 109.22) (width 0.5) (layer B.Cu) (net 13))
 (segment (start 180.848 109.22) (end 178.054 106.426) (width 0.5) (layer B.Cu) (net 13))
 (segment (start 178.054 106.426) (end 178.054 104.648) (width 0.5) (layer B.Cu) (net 13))
 (segment (start 178.054 104.648) (end 175.514 102.108) (width 0.5) (layer B.Cu) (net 13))
 (segment (start 175.514 102.108) (end 159.004 102.108) (width 0.5) (layer B.Cu) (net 13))
 (segment (start 159.004 102.108) (end 156.464 104.648) (width 0.5) (layer B.Cu) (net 13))
 (segment (start 156.464 104.648) (end 154.178 104.648) (width 0.5) (layer B.Cu) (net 13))
 (segment (start 154.178 104.648) (end 153.162 103.632) (width 0.5) (layer B.Cu) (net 13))
 (segment (start 153.162 103.632) (end 153.162 94.488) (width 0.5) (layer B.Cu) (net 13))
 (segment (start 153.162 94.488) (end 158.496 89.154) (width 0.5) (layer B.Cu) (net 13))
 (segment (start 158.496 89.154) (end 164.846 89.154) (width 0.5) (layer B.Cu) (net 13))
 (segment (start 174.579999 79.420001) (end 174.579999 76.118001) (width 0.5) (layer B.Cu) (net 13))
 (segment (start 164.846 89.154) (end 174.579999 79.420001) (width 0.5) (layer B.Cu) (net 13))
 (segment (start 174.579999 76.118001) (end 176.53 74.168) (width 0.5) (layer B.Cu) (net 13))
 (segment (start 183.380242 74.168) (end 185.41746 76.205218) (width 0.5) (layer B.Cu) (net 13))
 (segment (start 176.53 74.168) (end 183.380242 74.168) (width 0.5) (layer B.Cu) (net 13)))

